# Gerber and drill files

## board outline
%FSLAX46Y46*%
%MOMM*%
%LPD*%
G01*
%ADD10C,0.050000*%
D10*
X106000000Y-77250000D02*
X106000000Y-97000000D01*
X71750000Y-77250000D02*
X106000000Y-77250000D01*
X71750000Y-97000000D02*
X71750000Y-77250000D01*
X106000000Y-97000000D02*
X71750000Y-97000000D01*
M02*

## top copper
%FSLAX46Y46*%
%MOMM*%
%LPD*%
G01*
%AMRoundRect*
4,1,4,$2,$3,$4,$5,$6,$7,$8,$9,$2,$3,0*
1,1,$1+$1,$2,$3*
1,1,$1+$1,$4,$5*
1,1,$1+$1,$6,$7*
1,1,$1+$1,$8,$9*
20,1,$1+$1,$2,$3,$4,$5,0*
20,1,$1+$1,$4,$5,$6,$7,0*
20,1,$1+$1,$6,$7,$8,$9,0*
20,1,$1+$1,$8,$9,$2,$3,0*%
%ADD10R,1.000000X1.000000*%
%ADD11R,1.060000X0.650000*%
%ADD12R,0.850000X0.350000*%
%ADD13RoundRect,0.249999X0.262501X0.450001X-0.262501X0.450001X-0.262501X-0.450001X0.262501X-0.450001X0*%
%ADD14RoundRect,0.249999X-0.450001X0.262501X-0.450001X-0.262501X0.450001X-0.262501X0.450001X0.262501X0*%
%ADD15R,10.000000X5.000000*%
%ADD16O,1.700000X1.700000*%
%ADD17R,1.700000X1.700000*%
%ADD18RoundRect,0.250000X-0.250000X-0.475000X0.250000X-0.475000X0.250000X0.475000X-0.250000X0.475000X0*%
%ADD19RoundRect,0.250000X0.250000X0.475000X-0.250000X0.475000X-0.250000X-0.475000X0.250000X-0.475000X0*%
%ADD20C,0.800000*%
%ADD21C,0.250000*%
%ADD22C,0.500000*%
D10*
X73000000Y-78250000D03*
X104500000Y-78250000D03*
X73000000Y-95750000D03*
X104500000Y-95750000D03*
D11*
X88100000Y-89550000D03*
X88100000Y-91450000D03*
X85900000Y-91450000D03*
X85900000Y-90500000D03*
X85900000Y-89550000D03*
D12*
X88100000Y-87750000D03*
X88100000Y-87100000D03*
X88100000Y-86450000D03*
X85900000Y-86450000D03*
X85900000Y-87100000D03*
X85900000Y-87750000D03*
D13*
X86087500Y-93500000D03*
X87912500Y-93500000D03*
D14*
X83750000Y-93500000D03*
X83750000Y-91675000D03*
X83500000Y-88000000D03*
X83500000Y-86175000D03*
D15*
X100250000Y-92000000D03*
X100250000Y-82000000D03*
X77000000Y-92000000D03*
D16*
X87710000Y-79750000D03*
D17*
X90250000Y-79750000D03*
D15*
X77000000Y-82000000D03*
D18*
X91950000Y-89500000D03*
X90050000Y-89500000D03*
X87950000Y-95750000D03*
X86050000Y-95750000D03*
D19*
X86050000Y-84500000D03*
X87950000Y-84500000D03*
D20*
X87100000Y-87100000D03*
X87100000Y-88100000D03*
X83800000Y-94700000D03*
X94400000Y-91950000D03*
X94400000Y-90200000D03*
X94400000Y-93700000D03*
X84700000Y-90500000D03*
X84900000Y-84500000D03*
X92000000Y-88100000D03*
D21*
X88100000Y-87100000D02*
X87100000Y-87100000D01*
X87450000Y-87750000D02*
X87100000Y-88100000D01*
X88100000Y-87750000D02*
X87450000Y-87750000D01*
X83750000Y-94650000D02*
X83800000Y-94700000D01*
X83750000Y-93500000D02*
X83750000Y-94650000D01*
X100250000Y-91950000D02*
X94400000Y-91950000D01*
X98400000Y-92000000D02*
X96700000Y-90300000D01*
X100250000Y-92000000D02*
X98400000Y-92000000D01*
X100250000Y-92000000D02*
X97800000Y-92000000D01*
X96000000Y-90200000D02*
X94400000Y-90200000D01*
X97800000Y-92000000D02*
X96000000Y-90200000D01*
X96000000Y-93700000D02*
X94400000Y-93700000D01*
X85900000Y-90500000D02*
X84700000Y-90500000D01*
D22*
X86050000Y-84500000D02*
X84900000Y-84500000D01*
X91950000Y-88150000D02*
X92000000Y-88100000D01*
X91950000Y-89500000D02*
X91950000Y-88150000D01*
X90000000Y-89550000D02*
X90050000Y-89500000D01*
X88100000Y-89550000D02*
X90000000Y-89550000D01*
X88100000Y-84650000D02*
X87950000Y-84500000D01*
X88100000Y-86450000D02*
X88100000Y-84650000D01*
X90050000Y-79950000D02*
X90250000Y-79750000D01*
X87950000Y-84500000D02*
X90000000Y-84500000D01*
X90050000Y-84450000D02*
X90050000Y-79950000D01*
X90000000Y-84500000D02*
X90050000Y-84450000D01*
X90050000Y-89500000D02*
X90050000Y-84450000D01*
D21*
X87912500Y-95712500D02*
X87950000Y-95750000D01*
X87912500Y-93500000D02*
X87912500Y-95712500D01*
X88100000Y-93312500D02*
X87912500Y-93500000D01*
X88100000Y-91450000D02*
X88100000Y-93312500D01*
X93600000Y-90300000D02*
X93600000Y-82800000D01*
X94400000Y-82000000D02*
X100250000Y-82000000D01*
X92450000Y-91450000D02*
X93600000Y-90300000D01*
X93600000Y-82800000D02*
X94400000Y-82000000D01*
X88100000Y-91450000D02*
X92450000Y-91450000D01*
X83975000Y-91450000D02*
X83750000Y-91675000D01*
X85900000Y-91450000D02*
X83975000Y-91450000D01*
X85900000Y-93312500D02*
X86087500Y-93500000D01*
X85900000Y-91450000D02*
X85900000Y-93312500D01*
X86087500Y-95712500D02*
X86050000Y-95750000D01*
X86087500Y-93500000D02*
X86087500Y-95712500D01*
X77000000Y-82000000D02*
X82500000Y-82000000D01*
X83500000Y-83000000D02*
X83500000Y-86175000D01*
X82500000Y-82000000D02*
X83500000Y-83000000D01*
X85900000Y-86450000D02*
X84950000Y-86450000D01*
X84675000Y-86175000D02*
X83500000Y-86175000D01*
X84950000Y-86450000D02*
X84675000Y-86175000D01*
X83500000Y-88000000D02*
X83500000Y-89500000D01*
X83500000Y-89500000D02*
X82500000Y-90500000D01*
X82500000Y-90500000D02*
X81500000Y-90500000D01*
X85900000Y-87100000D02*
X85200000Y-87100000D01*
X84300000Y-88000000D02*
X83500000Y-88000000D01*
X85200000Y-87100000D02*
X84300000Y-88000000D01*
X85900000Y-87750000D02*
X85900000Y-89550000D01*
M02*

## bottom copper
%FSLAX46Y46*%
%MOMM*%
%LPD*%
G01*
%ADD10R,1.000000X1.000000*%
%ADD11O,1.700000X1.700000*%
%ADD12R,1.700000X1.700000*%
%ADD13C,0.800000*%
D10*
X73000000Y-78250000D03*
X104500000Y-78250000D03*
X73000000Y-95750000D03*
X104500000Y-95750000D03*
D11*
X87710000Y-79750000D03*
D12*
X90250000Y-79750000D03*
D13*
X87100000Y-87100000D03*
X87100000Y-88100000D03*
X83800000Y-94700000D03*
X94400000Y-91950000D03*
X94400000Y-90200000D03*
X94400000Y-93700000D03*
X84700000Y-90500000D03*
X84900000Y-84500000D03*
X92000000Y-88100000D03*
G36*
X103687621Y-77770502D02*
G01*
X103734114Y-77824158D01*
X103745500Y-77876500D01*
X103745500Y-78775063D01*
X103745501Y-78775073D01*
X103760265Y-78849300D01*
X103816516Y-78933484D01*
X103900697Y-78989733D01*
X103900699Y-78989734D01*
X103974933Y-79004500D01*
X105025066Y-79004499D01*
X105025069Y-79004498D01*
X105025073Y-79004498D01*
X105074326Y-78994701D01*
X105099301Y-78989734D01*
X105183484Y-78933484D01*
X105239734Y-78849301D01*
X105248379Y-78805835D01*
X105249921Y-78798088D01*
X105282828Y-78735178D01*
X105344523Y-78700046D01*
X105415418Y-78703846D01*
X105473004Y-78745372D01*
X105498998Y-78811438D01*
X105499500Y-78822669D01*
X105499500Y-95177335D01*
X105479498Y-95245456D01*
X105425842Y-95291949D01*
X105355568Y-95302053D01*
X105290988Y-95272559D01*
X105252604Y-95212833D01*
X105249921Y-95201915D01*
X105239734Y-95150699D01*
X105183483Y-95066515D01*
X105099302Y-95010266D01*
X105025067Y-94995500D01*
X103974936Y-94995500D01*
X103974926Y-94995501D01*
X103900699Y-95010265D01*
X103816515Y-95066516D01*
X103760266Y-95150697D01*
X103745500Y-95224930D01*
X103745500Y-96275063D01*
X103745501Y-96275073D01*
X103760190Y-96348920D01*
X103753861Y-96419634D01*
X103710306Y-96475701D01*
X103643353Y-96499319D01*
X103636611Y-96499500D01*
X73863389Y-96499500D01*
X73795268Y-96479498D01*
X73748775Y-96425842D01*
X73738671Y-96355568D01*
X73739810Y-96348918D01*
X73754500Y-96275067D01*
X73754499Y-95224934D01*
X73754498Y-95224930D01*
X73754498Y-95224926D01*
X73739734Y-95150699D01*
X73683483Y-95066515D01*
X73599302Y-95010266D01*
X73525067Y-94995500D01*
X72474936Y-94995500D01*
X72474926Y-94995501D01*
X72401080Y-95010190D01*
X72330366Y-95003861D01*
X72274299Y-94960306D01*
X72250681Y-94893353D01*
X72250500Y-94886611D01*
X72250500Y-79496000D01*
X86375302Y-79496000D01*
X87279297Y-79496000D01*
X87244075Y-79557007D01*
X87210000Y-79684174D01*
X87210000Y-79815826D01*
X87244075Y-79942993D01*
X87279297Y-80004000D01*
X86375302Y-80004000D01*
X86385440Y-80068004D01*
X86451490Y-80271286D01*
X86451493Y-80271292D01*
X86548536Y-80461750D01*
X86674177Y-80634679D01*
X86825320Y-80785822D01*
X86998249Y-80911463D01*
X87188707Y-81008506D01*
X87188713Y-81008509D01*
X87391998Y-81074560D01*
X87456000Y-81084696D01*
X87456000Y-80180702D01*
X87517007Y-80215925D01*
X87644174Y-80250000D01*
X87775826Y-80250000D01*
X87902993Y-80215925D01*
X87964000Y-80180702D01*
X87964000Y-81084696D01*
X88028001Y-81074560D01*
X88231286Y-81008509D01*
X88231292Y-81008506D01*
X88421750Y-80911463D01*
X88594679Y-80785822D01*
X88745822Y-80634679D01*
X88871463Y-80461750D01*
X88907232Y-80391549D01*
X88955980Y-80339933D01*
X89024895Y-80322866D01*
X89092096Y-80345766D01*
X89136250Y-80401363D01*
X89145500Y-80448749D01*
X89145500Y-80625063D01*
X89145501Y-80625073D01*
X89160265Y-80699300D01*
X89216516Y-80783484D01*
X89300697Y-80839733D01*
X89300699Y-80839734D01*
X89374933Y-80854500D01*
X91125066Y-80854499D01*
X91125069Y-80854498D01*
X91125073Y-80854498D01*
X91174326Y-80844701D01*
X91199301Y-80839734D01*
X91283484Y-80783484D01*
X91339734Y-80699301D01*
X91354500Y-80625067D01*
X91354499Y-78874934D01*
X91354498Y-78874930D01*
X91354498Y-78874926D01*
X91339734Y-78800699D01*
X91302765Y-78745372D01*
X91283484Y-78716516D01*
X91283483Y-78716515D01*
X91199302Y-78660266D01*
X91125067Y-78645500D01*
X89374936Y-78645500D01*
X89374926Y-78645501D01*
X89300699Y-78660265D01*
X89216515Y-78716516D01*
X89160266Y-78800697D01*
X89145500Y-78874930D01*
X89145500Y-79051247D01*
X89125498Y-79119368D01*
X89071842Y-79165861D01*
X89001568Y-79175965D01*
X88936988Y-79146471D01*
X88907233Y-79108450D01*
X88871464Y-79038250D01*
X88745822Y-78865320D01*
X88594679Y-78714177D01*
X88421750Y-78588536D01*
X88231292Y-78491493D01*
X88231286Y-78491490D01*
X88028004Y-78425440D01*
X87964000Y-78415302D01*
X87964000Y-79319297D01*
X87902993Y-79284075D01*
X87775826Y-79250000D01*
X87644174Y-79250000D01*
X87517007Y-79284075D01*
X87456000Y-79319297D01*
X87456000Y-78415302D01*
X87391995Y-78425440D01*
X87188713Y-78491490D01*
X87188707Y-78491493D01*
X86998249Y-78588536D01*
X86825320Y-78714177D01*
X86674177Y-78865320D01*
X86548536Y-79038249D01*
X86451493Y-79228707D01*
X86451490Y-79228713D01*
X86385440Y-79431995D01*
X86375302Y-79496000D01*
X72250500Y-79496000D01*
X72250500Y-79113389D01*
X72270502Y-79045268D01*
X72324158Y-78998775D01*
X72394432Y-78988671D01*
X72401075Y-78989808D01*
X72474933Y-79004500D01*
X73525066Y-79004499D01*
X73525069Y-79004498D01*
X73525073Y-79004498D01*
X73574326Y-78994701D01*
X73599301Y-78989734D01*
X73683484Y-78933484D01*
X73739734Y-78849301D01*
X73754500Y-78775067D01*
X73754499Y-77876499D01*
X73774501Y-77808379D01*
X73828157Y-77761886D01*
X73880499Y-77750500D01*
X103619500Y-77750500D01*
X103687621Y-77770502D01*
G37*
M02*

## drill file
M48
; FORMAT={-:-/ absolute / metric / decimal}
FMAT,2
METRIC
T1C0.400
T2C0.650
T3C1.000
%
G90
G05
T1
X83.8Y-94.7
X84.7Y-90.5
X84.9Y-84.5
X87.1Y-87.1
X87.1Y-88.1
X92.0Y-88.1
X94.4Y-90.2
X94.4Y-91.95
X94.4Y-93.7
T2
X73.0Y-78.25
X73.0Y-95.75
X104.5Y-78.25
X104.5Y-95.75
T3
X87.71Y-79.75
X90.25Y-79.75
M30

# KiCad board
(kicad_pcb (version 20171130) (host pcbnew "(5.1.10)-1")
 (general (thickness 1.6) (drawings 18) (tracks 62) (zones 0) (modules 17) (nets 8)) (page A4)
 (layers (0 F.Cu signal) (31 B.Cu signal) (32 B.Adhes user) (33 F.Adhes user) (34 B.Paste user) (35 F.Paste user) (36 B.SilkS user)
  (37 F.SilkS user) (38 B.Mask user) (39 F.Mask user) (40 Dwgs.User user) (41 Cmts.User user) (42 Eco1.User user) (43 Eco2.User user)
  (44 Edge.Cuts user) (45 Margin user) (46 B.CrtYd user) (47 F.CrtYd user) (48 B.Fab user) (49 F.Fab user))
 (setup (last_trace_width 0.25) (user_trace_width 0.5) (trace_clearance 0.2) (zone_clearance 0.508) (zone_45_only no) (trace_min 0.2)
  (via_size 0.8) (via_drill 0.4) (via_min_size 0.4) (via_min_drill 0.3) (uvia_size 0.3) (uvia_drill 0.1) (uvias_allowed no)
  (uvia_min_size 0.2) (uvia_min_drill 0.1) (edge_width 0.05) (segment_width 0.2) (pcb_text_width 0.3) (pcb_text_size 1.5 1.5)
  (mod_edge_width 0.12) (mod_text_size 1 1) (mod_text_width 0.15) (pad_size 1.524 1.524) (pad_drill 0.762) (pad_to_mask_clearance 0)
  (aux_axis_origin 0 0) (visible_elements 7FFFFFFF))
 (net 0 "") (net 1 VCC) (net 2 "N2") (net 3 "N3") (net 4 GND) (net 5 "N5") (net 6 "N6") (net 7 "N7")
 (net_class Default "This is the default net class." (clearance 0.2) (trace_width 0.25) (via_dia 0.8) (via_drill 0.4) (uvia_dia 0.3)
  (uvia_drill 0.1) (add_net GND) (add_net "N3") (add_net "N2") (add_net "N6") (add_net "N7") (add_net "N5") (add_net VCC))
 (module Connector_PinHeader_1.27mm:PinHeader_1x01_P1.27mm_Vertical (layer F.Cu) (at 73 78.25 180)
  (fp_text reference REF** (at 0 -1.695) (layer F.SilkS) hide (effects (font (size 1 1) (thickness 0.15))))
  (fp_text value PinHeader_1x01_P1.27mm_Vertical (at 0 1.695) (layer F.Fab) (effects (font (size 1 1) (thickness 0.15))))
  (pad 1 thru_hole rect (at 0 0 180) (size 1 1) (drill 0.65) (layers *.Cu *.Mask)))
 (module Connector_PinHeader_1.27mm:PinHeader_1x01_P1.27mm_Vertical (layer F.Cu) (at 104.5 78.25)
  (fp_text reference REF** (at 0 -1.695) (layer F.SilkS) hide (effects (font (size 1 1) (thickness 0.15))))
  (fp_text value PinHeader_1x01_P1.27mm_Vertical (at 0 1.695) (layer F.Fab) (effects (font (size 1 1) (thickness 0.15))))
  (pad 1 thru_hole rect (at 0 0) (size 1 1) (drill 0.65) (layers *.Cu *.Mask)))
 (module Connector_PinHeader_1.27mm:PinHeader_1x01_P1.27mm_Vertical (layer F.Cu) (at 73 95.75 180)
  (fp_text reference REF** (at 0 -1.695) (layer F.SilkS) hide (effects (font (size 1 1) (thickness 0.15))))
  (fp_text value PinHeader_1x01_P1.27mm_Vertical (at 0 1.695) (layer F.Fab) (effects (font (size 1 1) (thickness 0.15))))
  (pad 1 thru_hole rect (at 0 0 180) (size 1 1) (drill 0.65) (layers *.Cu *.Mask)))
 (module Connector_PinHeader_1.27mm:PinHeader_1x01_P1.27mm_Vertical (layer F.Cu) (at 104.5 95.75)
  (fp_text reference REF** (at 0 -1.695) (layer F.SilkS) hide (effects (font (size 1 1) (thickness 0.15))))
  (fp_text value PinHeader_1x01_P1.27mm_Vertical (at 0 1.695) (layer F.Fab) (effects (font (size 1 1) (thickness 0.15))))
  (pad 1 thru_hole rect (at 0 0) (size 1 1) (drill 0.65) (layers *.Cu *.Mask)))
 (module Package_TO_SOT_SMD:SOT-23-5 (layer F.Cu) (at 87 90.5)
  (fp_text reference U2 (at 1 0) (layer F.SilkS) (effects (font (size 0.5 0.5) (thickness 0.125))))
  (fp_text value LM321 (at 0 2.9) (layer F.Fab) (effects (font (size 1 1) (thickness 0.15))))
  (pad 5 smd rect (at 1.1 -0.95) (size 1.06 0.65) (layers F.Cu F.Paste F.Mask) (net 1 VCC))
  (pad 4 smd rect (at 1.1 0.95) (size 1.06 0.65) (layers F.Cu F.Paste F.Mask) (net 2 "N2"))
  (pad 3 smd rect (at -1.1 0.95) (size 1.06 0.65) (layers F.Cu F.Paste F.Mask) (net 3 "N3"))
  (pad 2 smd rect (at -1.1 0) (size 1.06 0.65) (layers F.Cu F.Paste F.Mask) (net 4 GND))
  (pad 1 smd rect (at -1.1 -0.95) (size 1.06 0.65) (layers F.Cu F.Paste F.Mask) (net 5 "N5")))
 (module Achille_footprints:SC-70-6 (layer F.Cu) (at 87 87 180)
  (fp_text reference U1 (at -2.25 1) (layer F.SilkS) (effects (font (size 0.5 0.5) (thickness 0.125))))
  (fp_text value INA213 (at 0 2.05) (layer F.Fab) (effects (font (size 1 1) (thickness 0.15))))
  (pad 1 smd rect (at -1.1 -0.75 90) (size 0.35 0.85) (layers F.Cu F.Paste F.Mask) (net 4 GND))
  (pad 2 smd rect (at -1.1 -0.1 90) (size 0.35 0.85) (layers F.Cu F.Paste F.Mask) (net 4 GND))
  (pad 3 smd rect (at -1.1 0.55 90) (size 0.35 0.85) (layers F.Cu F.Paste F.Mask) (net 1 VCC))
  (pad 4 smd rect (at 1.1 0.55 90) (size 0.35 0.85) (layers F.Cu F.Paste F.Mask) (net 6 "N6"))
  (pad 5 smd rect (at 1.1 -0.1 90) (size 0.35 0.85) (layers F.Cu F.Paste F.Mask) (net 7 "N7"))
  (pad 6 smd rect (at 1.1 -0.75 90) (size 0.35 0.85) (layers F.Cu F.Paste F.Mask) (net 5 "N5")))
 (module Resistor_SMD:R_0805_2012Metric (layer F.Cu) (at 87 93.5 180)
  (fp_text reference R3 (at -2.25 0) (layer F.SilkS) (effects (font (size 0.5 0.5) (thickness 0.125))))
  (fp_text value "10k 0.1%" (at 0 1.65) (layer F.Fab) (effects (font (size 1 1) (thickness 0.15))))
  (pad 2 smd roundrect (at 0.9125 0 180) (size 1.025 1.4) (layers F.Cu F.Paste F.Mask) (roundrect_rratio 0.2439014634146341) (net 3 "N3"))
  (pad 1 smd roundrect (at -0.9125 0 180) (size 1.025 1.4) (layers F.Cu F.Paste F.Mask) (roundrect_rratio 0.2439014634146341) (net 2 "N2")))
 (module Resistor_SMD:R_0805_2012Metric (layer F.Cu) (at 83.75 92.5875 270)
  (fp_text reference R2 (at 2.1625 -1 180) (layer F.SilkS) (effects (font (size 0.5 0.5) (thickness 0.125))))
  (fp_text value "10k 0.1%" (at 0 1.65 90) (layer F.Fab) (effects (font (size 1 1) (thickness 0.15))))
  (pad 2 smd roundrect (at 0.9125 0 270) (size 1.025 1.4) (layers F.Cu F.Paste F.Mask) (roundrect_rratio 0.2439014634146341) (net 4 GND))
  (pad 1 smd roundrect (at -0.9125 0 270) (size 1.025 1.4) (layers F.Cu F.Paste F.Mask) (roundrect_rratio 0.2439014634146341) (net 3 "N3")))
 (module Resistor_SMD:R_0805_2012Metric (layer F.Cu) (at 83.5 87.0875 270)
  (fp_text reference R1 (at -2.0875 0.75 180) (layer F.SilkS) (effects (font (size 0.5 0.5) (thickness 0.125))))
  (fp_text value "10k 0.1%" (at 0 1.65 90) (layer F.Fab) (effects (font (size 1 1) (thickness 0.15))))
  (pad 2 smd roundrect (at 0.9125 0 270) (size 1.025 1.4) (layers F.Cu F.Paste F.Mask) (roundrect_rratio 0.2439014634146341) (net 7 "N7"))
  (pad 1 smd roundrect (at -0.9125 0 270) (size 1.025 1.4) (layers F.Cu F.Paste F.Mask) (roundrect_rratio 0.2439014634146341) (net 6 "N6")))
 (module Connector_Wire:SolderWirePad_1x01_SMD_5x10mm (layer F.Cu) (at 100.25 92 90)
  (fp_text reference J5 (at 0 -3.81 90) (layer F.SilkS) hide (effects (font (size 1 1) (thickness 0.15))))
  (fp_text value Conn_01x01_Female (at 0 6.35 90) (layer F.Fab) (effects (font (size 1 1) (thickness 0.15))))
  (pad 1 smd rect (at 0 0 90) (size 5 10) (layers F.Cu F.Paste F.Mask) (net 4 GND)))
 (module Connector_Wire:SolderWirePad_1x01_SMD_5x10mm (layer F.Cu) (at 100.25 82 90)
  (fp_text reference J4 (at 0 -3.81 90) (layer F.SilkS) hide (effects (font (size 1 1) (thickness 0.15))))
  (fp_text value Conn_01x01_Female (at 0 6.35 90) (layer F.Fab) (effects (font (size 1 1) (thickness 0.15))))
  (pad 1 smd rect (at 0 0 90) (size 5 10) (layers F.Cu F.Paste F.Mask) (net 2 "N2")))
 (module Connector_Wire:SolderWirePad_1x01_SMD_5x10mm (layer F.Cu) (at 77 92 90)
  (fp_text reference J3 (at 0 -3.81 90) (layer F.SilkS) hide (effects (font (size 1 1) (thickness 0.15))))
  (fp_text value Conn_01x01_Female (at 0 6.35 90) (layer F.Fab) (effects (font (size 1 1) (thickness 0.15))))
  (pad 1 smd rect (at 0 0 90) (size 5 10) (layers F.Cu F.Paste F.Mask) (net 7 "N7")))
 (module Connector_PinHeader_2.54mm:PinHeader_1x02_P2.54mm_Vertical (layer F.Cu) (at 90.25 79.75 270)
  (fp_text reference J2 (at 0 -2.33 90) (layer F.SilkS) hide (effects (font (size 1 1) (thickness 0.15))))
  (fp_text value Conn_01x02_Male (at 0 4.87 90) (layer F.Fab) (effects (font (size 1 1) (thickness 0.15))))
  (pad 2 thru_hole oval (at 0 2.54 270) (size 1.7 1.7) (drill 1) (layers *.Cu *.Mask) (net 4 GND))
  (pad 1 thru_hole rect (at 0 0 270) (size 1.7 1.7) (drill 1) (layers *.Cu *.Mask) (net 1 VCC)))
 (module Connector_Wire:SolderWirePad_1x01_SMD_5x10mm (layer F.Cu) (at 77 82 90)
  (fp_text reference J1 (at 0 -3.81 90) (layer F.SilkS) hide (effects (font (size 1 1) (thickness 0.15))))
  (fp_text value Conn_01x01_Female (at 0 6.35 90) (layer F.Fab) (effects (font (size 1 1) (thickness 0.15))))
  (pad 1 smd rect (at 0 0 90) (size 5 10) (layers F.Cu F.Paste F.Mask) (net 6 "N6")))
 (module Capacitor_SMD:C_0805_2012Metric (layer F.Cu) (at 91 89.5)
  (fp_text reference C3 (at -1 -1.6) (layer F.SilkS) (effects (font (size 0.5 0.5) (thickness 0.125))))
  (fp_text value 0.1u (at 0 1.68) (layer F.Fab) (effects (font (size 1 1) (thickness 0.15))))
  (pad 2 smd roundrect (at 0.95 0) (size 1 1.45) (layers F.Cu F.Paste F.Mask) (roundrect_rratio 0.25) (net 4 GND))
  (pad 1 smd roundrect (at -0.95 0) (size 1 1.45) (layers F.Cu F.Paste F.Mask) (roundrect_rratio 0.25) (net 1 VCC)))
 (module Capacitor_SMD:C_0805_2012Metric (layer F.Cu) (at 87 95.75)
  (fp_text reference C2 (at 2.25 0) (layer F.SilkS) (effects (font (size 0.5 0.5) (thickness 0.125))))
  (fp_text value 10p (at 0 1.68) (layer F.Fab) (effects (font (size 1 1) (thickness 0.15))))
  (pad 2 smd roundrect (at 0.95 0) (size 1 1.45) (layers F.Cu F.Paste F.Mask) (roundrect_rratio 0.25) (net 2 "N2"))
  (pad 1 smd roundrect (at -0.95 0) (size 1 1.45) (layers F.Cu F.Paste F.Mask) (roundrect_rratio 0.25) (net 3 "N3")))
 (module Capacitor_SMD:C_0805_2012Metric (layer F.Cu) (at 87 84.5 180)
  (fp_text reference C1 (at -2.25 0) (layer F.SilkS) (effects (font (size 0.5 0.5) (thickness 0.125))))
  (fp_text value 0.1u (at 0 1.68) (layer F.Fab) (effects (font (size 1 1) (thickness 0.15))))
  (pad 2 smd roundrect (at 0.95 0 180) (size 1 1.45) (layers F.Cu F.Paste F.Mask) (roundrect_rratio 0.25) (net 4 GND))
  (pad 1 smd roundrect (at -0.95 0 180) (size 1 1.45) (layers F.Cu F.Paste F.Mask) (roundrect_rratio 0.25) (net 1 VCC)))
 (gr_line (start 106 77.25) (end 106 97) (layer Edge.Cuts) (width 0.05))
 (gr_line (start 71.75 77.25) (end 106 77.25) (layer Edge.Cuts) (width 0.05))
 (gr_line (start 71.75 97) (end 71.75 77.25) (layer Edge.Cuts) (width 0.05))
 (gr_line (start 106 97) (end 71.75 97) (layer Edge.Cuts) (width 0.05))
 (via (at 87.1 87.1) (size 0.8) (drill 0.4) (layers F.Cu B.Cu) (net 4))
 (segment (start 88.1 87.1) (end 87.1 87.1) (width 0.25) (layer F.Cu) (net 4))
 (via (at 87.1 88.1) (size 0.8) (drill 0.4) (layers F.Cu B.Cu) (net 4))
 (segment (start 87.45 87.75) (end 87.1 88.1) (width 0.25) (layer F.Cu) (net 4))
 (segment (start 88.1 87.75) (end 87.45 87.75) (width 0.25) (layer F.Cu) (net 4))
 (via (at 83.8 94.7) (size 0.8) (drill 0.4) (layers F.Cu B.Cu) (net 4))
 (segment (start 83.75 94.65) (end 83.8 94.7) (width 0.25) (layer F.Cu) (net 4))
 (segment (start 83.75 93.5) (end 83.75 94.65) (width 0.25) (layer F.Cu) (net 4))
 (via (at 94.4 91.95) (size 0.8) (drill 0.4) (layers F.Cu B.Cu) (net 4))
 (segment (start 100.25 91.95) (end 94.4 91.95) (width 0.25) (layer F.Cu) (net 4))
 (segment (start 98.4 92) (end 96.7 90.3) (width 0.25) (layer F.Cu) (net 4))
 (segment (start 100.25 92) (end 98.4 92) (width 0.25) (layer F.Cu) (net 4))
 (segment (start 100.25 92) (end 97.8 92) (width 0.25) (layer F.Cu) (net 4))
 (via (at 94.4 90.2) (size 0.8) (drill 0.4) (layers F.Cu B.Cu) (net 4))
 (segment (start 96 90.2) (end 94.4 90.2) (width 0.25) (layer F.Cu) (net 4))
 (segment (start 97.8 92) (end 96 90.2) (width 0.25) (layer F.Cu) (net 4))
 (segment (start 96 93.7) (end 94.4 93.7) (width 0.25) (layer F.Cu) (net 4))
 (via (at 94.4 93.7) (size 0.8) (drill 0.4) (layers F.Cu B.Cu) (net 4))
 (via (at 84.7 90.5) (size 0.8) (drill 0.4) (layers F.Cu B.Cu) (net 4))
 (segment (start 85.9 90.5) (end 84.7 90.5) (width 0.25) (layer F.Cu) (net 4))
 (via (at 84.9 84.5) (size 0.8) (drill 0.4) (layers F.Cu B.Cu) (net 4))
 (segment (start 86.05 84.5) (end 84.9 84.5) (width 0.5) (layer F.Cu) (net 4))
 (segment (start 91.95 88.15) (end 92 88.1) (width 0.5) (layer F.Cu) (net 4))
 (via (at 92 88.1) (size 0.8) (drill 0.4) (layers F.Cu B.Cu) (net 4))
 (segment (start 91.95 89.5) (end 91.95 88.15) (width 0.5) (layer F.Cu) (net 4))
 (segment (start 90 89.55) (end 90.05 89.5) (width 0.5) (layer F.Cu) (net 1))
 (segment (start 88.1 89.55) (end 90 89.55) (width 0.5) (layer F.Cu) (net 1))
 (segment (start 88.1 84.65) (end 87.95 84.5) (width 0.5) (layer F.Cu) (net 1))
 (segment (start 88.1 86.45) (end 88.1 84.65) (width 0.5) (layer F.Cu) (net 1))
 (segment (start 90.05 79.95) (end 90.25 79.75) (width 0.5) (layer F.Cu) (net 1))
 (segment (start 87.95 84.5) (end 90 84.5) (width 0.5) (layer F.Cu) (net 1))
 (segment (start 90.05 84.45) (end 90.05 79.95) (width 0.5) (layer F.Cu) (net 1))
 (segment (start 90 84.5) (end 90.05 84.45) (width 0.5) (layer F.Cu) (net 1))
 (segment (start 90.05 89.5) (end 90.05 84.45) (width 0.5) (layer F.Cu) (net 1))
 (segment (start 87.9125 95.7125) (end 87.95 95.75) (width 0.25) (layer F.Cu) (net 2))
 (segment (start 87.9125 93.5) (end 87.9125 95.7125) (width 0.25) (layer F.Cu) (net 2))
 (segment (start 88.1 93.3125) (end 87.9125 93.5) (width 0.25) (layer F.Cu) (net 2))
 (segment (start 88.1 91.45) (end 88.1 93.3125) (width 0.25) (layer F.Cu) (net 2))
 (segment (start 93.6 90.3) (end 93.6 82.8) (width 0.25) (layer F.Cu) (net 2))
 (segment (start 94.4 82) (end 100.25 82) (width 0.25) (layer F.Cu) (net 2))
 (segment (start 92.45 91.45) (end 93.6 90.3) (width 0.25) (layer F.Cu) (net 2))
 (segment (start 93.6 82.8) (end 94.4 82) (width 0.25) (layer F.Cu) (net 2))
 (segment (start 88.1 91.45) (end 92.45 91.45) (width 0.25) (layer F.Cu) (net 2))
 (segment (start 83.975 91.45) (end 83.75 91.675) (width 0.25) (layer F.Cu) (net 3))
 (segment (start 85.9 91.45) (end 83.975 91.45) (width 0.25) (layer F.Cu) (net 3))
 (segment (start 85.9 93.3125) (end 86.0875 93.5) (width 0.25) (layer F.Cu) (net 3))
 (segment (start 85.9 91.45) (end 85.9 93.3125) (width 0.25) (layer F.Cu) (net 3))
 (segment (start 86.0875 95.7125) (end 86.05 95.75) (width 0.25) (layer F.Cu) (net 3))
 (segment (start 86.0875 93.5) (end 86.0875 95.7125) (width 0.25) (layer F.Cu) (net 3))
 (segment (start 77 82) (end 82.5 82) (width 0.25) (layer F.Cu) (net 6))
 (segment (start 83.5 83) (end 83.5 86.175) (width 0.25) (layer F.Cu) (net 6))
 (segment (start 82.5 82) (end 83.5 83) (width 0.25) (layer F.Cu) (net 6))
 (segment (start 85.9 86.45) (end 84.95 86.45) (width 0.25) (layer F.Cu) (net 6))
 (segment (start 84.675 86.175) (end 83.5 86.175) (width 0.25) (layer F.Cu) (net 6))
 (segment (start 84.95 86.45) (end 84.675 86.175) (width 0.25) (layer F.Cu) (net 6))
 (segment (start 83.5 88) (end 83.5 89.5) (width 0.25) (layer F.Cu) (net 7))
 (segment (start 83.5 89.5) (end 82.5 90.5) (width 0.25) (layer F.Cu) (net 7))
 (segment (start 82.5 90.5) (end 81.5 90.5) (width 0.25) (layer F.Cu) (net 7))
 (segment (start 85.9 87.1) (end 85.2 87.1) (width 0.25) (layer F.Cu) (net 7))
 (segment (start 84.3 88) (end 83.5 88) (width 0.25) (layer F.Cu) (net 7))
 (segment (start 85.2 87.1) (end 84.3 88) (width 0.25) (layer F.Cu) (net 7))
 (segment (start 85.9 87.75) (end 85.9 89.55) (width 0.25) (layer F.Cu) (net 5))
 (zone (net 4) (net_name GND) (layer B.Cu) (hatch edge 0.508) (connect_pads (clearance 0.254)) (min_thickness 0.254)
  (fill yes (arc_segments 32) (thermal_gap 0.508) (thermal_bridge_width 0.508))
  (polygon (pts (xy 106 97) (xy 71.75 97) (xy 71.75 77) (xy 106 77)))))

